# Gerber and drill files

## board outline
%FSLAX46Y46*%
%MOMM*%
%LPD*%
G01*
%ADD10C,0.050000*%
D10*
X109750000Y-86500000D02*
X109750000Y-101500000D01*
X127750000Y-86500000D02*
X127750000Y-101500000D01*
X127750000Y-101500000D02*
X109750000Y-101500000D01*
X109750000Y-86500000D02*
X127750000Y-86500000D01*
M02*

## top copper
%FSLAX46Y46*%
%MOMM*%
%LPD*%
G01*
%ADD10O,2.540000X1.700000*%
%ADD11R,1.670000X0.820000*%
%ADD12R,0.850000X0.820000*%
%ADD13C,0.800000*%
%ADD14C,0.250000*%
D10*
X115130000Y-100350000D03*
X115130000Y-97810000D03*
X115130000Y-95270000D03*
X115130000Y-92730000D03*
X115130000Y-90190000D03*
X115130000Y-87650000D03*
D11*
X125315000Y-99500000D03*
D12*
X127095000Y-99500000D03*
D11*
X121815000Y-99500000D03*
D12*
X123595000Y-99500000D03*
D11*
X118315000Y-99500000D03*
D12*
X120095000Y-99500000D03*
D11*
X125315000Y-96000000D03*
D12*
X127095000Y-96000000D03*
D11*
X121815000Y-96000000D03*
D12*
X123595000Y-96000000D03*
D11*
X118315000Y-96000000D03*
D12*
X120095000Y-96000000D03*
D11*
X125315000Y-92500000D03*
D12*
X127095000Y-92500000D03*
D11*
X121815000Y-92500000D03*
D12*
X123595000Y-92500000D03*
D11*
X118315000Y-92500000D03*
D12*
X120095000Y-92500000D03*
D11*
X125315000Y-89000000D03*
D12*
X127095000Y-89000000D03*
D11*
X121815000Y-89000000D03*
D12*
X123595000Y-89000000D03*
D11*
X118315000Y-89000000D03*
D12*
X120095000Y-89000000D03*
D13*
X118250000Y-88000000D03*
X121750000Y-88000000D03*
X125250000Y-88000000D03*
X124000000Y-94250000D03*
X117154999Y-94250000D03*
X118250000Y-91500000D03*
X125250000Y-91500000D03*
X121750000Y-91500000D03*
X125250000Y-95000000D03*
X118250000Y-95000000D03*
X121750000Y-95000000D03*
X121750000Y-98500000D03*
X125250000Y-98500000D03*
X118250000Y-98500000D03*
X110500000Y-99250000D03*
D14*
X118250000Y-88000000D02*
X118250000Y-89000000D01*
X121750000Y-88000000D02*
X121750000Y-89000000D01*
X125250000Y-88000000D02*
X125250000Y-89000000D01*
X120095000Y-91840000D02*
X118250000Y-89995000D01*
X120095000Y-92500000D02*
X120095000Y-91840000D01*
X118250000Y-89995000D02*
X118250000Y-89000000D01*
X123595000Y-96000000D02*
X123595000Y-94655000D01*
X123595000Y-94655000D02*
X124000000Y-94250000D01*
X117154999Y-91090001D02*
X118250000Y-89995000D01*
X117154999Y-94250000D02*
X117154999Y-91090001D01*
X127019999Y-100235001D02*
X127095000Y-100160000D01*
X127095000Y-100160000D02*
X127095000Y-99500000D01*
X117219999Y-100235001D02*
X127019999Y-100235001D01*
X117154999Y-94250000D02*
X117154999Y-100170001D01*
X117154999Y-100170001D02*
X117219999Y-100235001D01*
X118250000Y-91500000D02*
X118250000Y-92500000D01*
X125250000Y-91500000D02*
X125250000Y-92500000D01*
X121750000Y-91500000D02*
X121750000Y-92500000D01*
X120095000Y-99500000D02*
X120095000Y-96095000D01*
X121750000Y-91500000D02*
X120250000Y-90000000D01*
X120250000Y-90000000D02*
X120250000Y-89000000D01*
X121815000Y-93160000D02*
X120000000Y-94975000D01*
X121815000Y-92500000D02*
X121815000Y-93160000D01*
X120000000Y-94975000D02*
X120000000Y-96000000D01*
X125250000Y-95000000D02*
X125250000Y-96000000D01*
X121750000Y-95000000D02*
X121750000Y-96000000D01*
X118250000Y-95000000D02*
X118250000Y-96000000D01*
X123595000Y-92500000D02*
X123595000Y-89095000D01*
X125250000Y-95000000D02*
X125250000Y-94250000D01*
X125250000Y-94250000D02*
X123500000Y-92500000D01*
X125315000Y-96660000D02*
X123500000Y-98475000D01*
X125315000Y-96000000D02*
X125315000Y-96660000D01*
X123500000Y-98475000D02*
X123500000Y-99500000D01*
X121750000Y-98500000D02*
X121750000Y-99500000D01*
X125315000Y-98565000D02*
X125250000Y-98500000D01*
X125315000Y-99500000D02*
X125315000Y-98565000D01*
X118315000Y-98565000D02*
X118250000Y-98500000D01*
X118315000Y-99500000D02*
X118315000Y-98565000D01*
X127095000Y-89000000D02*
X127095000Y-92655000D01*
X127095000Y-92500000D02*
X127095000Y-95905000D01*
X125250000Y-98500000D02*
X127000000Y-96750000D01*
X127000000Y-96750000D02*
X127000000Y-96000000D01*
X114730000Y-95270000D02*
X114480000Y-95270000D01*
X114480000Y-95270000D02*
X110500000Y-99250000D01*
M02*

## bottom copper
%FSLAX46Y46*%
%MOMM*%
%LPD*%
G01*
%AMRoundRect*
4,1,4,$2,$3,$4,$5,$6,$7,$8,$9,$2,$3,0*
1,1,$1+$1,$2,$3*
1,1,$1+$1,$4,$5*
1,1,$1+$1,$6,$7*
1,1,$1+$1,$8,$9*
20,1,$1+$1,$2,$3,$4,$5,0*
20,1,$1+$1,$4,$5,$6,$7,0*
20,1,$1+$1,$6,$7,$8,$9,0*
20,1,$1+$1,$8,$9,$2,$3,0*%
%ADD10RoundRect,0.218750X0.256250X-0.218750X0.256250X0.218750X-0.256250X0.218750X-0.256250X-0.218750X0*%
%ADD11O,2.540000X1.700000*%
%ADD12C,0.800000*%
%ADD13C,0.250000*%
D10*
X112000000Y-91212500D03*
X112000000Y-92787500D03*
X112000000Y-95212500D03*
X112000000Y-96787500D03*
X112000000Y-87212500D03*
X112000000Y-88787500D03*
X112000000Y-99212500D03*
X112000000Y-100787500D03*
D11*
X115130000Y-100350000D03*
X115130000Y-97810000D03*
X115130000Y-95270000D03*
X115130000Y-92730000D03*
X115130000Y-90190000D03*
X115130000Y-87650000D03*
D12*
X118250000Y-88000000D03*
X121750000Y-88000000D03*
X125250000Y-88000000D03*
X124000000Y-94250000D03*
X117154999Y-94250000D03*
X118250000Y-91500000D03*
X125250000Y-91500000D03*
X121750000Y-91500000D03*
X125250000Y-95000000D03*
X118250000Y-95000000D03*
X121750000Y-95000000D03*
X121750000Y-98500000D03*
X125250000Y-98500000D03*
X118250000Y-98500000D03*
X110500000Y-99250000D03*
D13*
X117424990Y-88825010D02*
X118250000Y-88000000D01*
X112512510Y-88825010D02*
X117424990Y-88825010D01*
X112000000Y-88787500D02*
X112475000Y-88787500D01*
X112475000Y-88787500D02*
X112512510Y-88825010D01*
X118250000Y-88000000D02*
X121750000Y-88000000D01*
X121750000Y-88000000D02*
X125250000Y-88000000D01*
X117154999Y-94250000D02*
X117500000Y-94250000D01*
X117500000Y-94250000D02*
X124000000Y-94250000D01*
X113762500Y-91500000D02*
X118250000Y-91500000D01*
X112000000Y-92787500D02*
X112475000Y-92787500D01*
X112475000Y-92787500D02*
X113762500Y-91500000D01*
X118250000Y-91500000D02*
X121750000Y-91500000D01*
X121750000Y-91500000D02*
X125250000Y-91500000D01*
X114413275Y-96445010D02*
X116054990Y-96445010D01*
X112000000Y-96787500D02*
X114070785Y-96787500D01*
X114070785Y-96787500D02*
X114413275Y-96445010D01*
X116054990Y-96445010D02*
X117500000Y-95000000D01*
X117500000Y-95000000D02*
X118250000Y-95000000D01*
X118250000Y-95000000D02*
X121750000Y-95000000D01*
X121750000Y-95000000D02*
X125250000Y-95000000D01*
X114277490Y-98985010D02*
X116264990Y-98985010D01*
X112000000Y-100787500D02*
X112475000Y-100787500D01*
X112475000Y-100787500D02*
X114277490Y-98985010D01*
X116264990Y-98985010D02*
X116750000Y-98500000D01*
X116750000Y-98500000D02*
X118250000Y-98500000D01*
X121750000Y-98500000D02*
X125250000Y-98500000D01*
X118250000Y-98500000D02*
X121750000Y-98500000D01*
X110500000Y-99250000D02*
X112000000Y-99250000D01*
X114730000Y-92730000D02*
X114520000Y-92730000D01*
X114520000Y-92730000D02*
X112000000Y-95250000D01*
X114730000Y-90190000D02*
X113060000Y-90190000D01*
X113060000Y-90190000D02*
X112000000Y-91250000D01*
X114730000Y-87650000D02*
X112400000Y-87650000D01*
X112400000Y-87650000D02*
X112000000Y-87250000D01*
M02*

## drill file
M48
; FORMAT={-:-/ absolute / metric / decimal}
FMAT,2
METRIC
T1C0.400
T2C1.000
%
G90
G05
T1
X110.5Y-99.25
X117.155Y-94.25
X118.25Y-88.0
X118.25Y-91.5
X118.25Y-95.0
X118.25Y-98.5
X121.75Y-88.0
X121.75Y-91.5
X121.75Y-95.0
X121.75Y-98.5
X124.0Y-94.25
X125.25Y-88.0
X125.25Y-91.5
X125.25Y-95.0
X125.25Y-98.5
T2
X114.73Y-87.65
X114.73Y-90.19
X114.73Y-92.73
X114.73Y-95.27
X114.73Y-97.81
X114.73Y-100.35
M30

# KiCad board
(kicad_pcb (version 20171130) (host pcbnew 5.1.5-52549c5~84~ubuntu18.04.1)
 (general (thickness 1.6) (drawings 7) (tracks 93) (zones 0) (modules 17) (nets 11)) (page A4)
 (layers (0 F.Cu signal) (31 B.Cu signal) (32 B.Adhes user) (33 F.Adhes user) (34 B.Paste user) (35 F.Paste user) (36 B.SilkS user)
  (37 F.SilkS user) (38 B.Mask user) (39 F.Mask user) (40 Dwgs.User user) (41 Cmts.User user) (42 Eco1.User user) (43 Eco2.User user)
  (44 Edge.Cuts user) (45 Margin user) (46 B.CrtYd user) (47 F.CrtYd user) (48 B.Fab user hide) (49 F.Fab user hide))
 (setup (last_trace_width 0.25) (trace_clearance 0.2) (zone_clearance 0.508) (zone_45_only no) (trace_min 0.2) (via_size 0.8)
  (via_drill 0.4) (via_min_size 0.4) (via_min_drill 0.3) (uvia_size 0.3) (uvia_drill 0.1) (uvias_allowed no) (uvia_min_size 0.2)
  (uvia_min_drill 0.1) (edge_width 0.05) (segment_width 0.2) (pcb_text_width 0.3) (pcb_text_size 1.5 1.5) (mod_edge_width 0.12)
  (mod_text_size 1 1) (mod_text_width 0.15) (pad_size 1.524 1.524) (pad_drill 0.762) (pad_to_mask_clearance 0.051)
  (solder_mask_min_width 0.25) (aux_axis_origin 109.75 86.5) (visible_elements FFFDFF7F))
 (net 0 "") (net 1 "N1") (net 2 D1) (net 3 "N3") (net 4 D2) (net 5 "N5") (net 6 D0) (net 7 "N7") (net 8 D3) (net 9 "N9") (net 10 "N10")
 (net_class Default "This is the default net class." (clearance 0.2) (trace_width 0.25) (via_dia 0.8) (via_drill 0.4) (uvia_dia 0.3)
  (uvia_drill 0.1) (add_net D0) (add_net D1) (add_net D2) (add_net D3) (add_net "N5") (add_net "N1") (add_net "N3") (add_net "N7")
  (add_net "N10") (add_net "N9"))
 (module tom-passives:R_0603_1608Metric (layer B.Cu) (at 112 92 90)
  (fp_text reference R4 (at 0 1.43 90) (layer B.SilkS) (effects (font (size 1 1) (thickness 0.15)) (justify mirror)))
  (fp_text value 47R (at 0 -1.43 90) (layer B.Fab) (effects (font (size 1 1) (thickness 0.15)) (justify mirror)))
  (pad 2 smd roundrect (at 0.7875 0 90) (size 0.875 0.95) (layers B.Cu B.Paste B.Mask) (roundrect_rratio 0.25) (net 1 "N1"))
  (pad 1 smd roundrect (at -0.7875 0 90) (size 0.875 0.95) (layers B.Cu B.Paste B.Mask) (roundrect_rratio 0.25) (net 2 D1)))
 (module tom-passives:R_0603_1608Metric (layer B.Cu) (at 112 96 90)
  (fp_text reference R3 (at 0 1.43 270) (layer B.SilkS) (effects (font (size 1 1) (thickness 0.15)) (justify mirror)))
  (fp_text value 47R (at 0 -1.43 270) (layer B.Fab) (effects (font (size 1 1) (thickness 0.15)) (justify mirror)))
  (pad 2 smd roundrect (at 0.7875 0 90) (size 0.875 0.95) (layers B.Cu B.Paste B.Mask) (roundrect_rratio 0.25) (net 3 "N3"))
  (pad 1 smd roundrect (at -0.7875 0 90) (size 0.875 0.95) (layers B.Cu B.Paste B.Mask) (roundrect_rratio 0.25) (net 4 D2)))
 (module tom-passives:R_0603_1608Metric (layer B.Cu) (at 112 88 90)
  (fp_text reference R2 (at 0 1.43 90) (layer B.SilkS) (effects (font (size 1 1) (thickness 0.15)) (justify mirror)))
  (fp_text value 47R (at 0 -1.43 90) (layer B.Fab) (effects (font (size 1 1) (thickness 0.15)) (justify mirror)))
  (pad 2 smd roundrect (at 0.7875 0 90) (size 0.875 0.95) (layers B.Cu B.Paste B.Mask) (roundrect_rratio 0.25) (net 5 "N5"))
  (pad 1 smd roundrect (at -0.7875 0 90) (size 0.875 0.95) (layers B.Cu B.Paste B.Mask) (roundrect_rratio 0.25) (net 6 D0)))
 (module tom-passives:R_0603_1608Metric (layer B.Cu) (at 112 100 90)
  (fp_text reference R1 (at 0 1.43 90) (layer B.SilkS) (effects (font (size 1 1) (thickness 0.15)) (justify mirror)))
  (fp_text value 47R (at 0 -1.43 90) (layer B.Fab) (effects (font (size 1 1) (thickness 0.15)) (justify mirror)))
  (pad 2 smd roundrect (at 0.7875 0 90) (size 0.875 0.95) (layers B.Cu B.Paste B.Mask) (roundrect_rratio 0.25) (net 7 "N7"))
  (pad 1 smd roundrect (at -0.7875 0 90) (size 0.875 0.95) (layers B.Cu B.Paste B.Mask) (roundrect_rratio 0.25) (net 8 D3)))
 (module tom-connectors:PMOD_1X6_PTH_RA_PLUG (layer F.Cu) (at 116 94 270)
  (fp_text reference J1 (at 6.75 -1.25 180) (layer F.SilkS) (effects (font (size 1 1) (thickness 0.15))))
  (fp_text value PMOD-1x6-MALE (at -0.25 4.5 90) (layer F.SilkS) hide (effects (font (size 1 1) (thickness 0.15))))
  (pad 6 thru_hole oval (at 6.35 1.27 180) (size 2.54 1.7) (drill 1 (offset -0.4 0)) (layers *.Cu *.Mask) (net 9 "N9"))
  (pad 5 thru_hole oval (at 3.81 1.27 180) (size 2.54 1.7) (drill 1 (offset -0.4 0)) (layers *.Cu *.Mask) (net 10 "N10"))
  (pad 4 thru_hole oval (at 1.27 1.27 180) (size 2.54 1.7) (drill 1 (offset -0.4 0)) (layers *.Cu *.Mask) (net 7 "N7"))
  (pad 3 thru_hole oval (at -1.27 1.27 180) (size 2.54 1.7) (drill 1 (offset -0.4 0)) (layers *.Cu *.Mask) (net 3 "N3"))
  (pad 2 thru_hole oval (at -3.81 1.27 180) (size 2.54 1.7) (drill 1 (offset -0.4 0)) (layers *.Cu *.Mask) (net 1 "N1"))
  (pad 1 thru_hole oval (at -6.35 1.27 180) (size 2.54 1.7) (drill 1 (offset -0.4 0)) (layers *.Cu *.Mask) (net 5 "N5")))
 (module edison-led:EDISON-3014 (layer F.Cu) (at 126 99.5)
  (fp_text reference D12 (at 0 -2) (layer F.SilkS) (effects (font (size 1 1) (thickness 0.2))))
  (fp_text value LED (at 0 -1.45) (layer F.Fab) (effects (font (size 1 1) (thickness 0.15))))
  (pad 2 smd rect (at -0.685 0) (size 1.67 0.82) (layers F.Cu F.Paste F.Mask) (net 8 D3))
  (pad 1 smd rect (at 1.095 0) (size 0.85 0.82) (layers F.Cu F.Paste F.Mask) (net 6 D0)))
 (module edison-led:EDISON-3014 (layer F.Cu) (at 122.5 99.5)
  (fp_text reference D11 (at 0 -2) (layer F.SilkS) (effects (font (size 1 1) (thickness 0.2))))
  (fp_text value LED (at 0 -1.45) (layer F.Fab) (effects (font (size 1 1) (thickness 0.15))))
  (pad 2 smd rect (at -0.685 0) (size 1.67 0.82) (layers F.Cu F.Paste F.Mask) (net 8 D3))
  (pad 1 smd rect (at 1.095 0) (size 0.85 0.82) (layers F.Cu F.Paste F.Mask) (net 4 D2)))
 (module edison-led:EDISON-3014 (layer F.Cu) (at 119 99.5)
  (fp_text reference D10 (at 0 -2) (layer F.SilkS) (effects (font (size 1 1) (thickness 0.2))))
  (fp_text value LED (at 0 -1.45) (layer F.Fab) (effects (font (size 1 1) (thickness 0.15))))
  (pad 2 smd rect (at -0.685 0) (size 1.67 0.82) (layers F.Cu F.Paste F.Mask) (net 8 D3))
  (pad 1 smd rect (at 1.095 0) (size 0.85 0.82) (layers F.Cu F.Paste F.Mask) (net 2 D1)))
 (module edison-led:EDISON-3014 (layer F.Cu) (at 126 96)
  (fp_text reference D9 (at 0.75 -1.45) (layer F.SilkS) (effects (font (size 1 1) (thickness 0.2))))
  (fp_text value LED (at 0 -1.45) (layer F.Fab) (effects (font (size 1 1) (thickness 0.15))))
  (pad 2 smd rect (at -0.685 0) (size 1.67 0.82) (layers F.Cu F.Paste F.Mask) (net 4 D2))
  (pad 1 smd rect (at 1.095 0) (size 0.85 0.82) (layers F.Cu F.Paste F.Mask) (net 8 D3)))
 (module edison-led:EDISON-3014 (layer F.Cu) (at 122.5 96)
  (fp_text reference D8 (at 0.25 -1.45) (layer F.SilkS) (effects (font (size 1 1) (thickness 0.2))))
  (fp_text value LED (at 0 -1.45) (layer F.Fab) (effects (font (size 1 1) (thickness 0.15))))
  (pad 2 smd rect (at -0.685 0) (size 1.67 0.82) (layers F.Cu F.Paste F.Mask) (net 4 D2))
  (pad 1 smd rect (at 1.095 0) (size 0.85 0.82) (layers F.Cu F.Paste F.Mask) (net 6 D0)))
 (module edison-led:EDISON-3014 (layer F.Cu) (at 119 96)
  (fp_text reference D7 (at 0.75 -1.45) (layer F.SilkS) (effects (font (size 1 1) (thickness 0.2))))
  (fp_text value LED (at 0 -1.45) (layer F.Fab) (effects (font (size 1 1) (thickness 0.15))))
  (pad 2 smd rect (at -0.685 0) (size 1.67 0.82) (layers F.Cu F.Paste F.Mask) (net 4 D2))
  (pad 1 smd rect (at 1.095 0) (size 0.85 0.82) (layers F.Cu F.Paste F.Mask) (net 2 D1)))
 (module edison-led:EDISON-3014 (layer F.Cu) (at 126 92.5)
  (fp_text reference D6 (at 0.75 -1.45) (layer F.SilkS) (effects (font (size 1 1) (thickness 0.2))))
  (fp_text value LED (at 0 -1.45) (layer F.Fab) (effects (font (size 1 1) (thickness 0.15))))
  (pad 2 smd rect (at -0.685 0) (size 1.67 0.82) (layers F.Cu F.Paste F.Mask) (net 2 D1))
  (pad 1 smd rect (at 1.095 0) (size 0.85 0.82) (layers F.Cu F.Paste F.Mask) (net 8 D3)))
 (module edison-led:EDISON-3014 (layer F.Cu) (at 122.5 92.5)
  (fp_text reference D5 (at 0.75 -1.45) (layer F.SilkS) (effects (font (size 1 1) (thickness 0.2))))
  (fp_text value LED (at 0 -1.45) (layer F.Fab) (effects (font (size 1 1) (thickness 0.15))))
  (pad 2 smd rect (at -0.685 0) (size 1.67 0.82) (layers F.Cu F.Paste F.Mask) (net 2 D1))
  (pad 1 smd rect (at 1.095 0) (size 0.85 0.82) (layers F.Cu F.Paste F.Mask) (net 4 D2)))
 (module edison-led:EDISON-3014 (layer F.Cu) (at 119 92.5)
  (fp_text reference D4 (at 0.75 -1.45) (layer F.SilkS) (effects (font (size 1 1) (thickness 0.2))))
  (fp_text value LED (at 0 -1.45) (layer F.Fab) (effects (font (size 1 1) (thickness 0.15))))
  (pad 2 smd rect (at -0.685 0) (size 1.67 0.82) (layers F.Cu F.Paste F.Mask) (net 2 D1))
  (pad 1 smd rect (at 1.095 0) (size 0.85 0.82) (layers F.Cu F.Paste F.Mask) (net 6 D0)))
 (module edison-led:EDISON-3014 (layer F.Cu) (at 126 89)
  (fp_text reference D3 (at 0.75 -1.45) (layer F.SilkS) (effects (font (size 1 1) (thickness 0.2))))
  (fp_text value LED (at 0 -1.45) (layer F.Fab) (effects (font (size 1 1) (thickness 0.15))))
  (pad 2 smd rect (at -0.685 0) (size 1.67 0.82) (layers F.Cu F.Paste F.Mask) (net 6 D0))
  (pad 1 smd rect (at 1.095 0) (size 0.85 0.82) (layers F.Cu F.Paste F.Mask) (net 8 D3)))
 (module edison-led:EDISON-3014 (layer F.Cu) (at 122.5 89)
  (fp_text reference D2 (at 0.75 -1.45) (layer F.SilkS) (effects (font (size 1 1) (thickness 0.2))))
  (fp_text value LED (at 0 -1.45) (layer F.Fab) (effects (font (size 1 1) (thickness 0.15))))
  (pad 2 smd rect (at -0.685 0) (size 1.67 0.82) (layers F.Cu F.Paste F.Mask) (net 6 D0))
  (pad 1 smd rect (at 1.095 0) (size 0.85 0.82) (layers F.Cu F.Paste F.Mask) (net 4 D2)))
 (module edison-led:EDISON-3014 (layer F.Cu) (at 119 89)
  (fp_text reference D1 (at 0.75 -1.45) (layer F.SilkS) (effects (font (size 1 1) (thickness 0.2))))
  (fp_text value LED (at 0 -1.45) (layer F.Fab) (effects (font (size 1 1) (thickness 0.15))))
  (pad 2 smd rect (at -0.685 0) (size 1.67 0.82) (layers F.Cu F.Paste F.Mask) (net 6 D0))
  (pad 1 smd rect (at 1.095 0) (size 0.85 0.82) (layers F.Cu F.Paste F.Mask) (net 2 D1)))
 (gr_line (start 109.75 86.5) (end 109.75 101.5) (layer Edge.Cuts) (width 0.05))
 (gr_line (start 127.75 86.5) (end 127.75 101.5) (layer Edge.Cuts) (width 0.05))
 (gr_line (start 127.75 101.5) (end 109.75 101.5) (layer Edge.Cuts) (width 0.05))
 (gr_line (start 109.75 86.5) (end 127.75 86.5) (layer Edge.Cuts) (width 0.05))
 (segment (start 117.42499 88.82501) (end 118.25 88) (width 0.25) (layer B.Cu) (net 6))
 (segment (start 112.51251 88.82501) (end 117.42499 88.82501) (width 0.25) (layer B.Cu) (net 6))
 (via (at 118.25 88) (size 0.8) (drill 0.4) (layers F.Cu B.Cu) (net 6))
 (segment (start 112 88.7875) (end 112.475 88.7875) (width 0.25) (layer B.Cu) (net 6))
 (segment (start 112.475 88.7875) (end 112.51251 88.82501) (width 0.25) (layer B.Cu) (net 6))
 (segment (start 118.25 88) (end 118.25 89) (width 0.25) (layer F.Cu) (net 6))
 (via (at 121.75 88) (size 0.8) (drill 0.4) (layers F.Cu B.Cu) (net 6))
 (segment (start 118.25 88) (end 121.75 88) (width 0.25) (layer B.Cu) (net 6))
 (segment (start 121.75 88) (end 121.75 89) (width 0.25) (layer F.Cu) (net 6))
 (via (at 125.25 88) (size 0.8) (drill 0.4) (layers F.Cu B.Cu) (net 6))
 (segment (start 121.75 88) (end 125.25 88) (width 0.25) (layer B.Cu) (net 6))
 (segment (start 125.25 88) (end 125.25 89) (width 0.25) (layer F.Cu) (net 6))
 (segment (start 120.095 91.84) (end 118.25 89.995) (width 0.25) (layer F.Cu) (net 6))
 (segment (start 120.095 92.5) (end 120.095 91.84) (width 0.25) (layer F.Cu) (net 6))
 (segment (start 118.25 89.995) (end 118.25 89) (width 0.25) (layer F.Cu) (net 6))
 (via (at 124 94.25) (size 0.8) (drill 0.4) (layers F.Cu B.Cu) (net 6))
 (segment (start 123.595 96) (end 123.595 94.655) (width 0.25) (layer F.Cu) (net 6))
 (segment (start 123.595 94.655) (end 124 94.25) (width 0.25) (layer F.Cu) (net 6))
 (segment (start 117.154999 91.090001) (end 118.25 89.995) (width 0.25) (layer F.Cu) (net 6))
 (segment (start 117.154999 94.25) (end 117.154999 91.090001) (width 0.25) (layer F.Cu) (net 6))
 (segment (start 127.019999 100.235001) (end 127.095 100.16) (width 0.25) (layer F.Cu) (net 6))
 (segment (start 117.154999 94.25) (end 117.5 94.25) (width 0.25) (layer B.Cu) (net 6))
 (via (at 117.154999 94.25) (size 0.8) (drill 0.4) (layers F.Cu B.Cu) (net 6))
 (segment (start 127.095 100.16) (end 127.095 99.5) (width 0.25) (layer F.Cu) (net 6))
 (segment (start 117.219999 100.235001) (end 127.019999 100.235001) (width 0.25) (layer F.Cu) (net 6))
 (segment (start 117.5 94.25) (end 124 94.25) (width 0.25) (layer B.Cu) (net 6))
 (segment (start 117.154999 94.25) (end 117.154999 100.170001) (width 0.25) (layer F.Cu) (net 6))
 (segment (start 117.154999 100.170001) (end 117.219999 100.235001) (width 0.25) (layer F.Cu) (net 6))
 (segment (start 113.7625 91.5) (end 118.25 91.5) (width 0.25) (layer B.Cu) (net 2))
 (segment (start 112 92.7875) (end 112.475 92.7875) (width 0.25) (layer B.Cu) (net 2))
 (via (at 118.25 91.5) (size 0.8) (drill 0.4) (layers F.Cu B.Cu) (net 2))
 (segment (start 112.475 92.7875) (end 113.7625 91.5) (width 0.25) (layer B.Cu) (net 2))
 (segment (start 118.25 91.5) (end 118.25 92.5) (width 0.25) (layer F.Cu) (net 2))
 (segment (start 118.25 91.5) (end 121.75 91.5) (width 0.25) (layer B.Cu) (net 2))
 (via (at 125.25 91.5) (size 0.8) (drill 0.4) (layers F.Cu B.Cu) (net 2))
 (segment (start 125.25 91.5) (end 125.25 92.5) (width 0.25) (layer F.Cu) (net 2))
 (segment (start 121.75 91.5) (end 125.25 91.5) (width 0.25) (layer B.Cu) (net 2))
 (via (at 121.75 91.5) (size 0.8) (drill 0.4) (layers F.Cu B.Cu) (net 2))
 (segment (start 121.75 91.5) (end 121.75 92.5) (width 0.25) (layer F.Cu) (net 2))
 (segment (start 120.095 99.5) (end 120.095 96.095) (width 0.25) (layer F.Cu) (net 2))
 (segment (start 121.75 91.5) (end 120.25 90) (width 0.25) (layer F.Cu) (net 2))
 (segment (start 120.25 90) (end 120.25 89) (width 0.25) (layer F.Cu) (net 2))
 (segment (start 121.815 93.16) (end 120 94.975) (width 0.25) (layer F.Cu) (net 2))
 (segment (start 121.815 92.5) (end 121.815 93.16) (width 0.25) (layer F.Cu) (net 2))
 (segment (start 120 94.975) (end 120 96) (width 0.25) (layer F.Cu) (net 2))
 (segment (start 114.413275 96.44501) (end 116.05499 96.44501) (width 0.25) (layer B.Cu) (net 4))
 (segment (start 112 96.7875) (end 114.070785 96.7875) (width 0.25) (layer B.Cu) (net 4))
 (segment (start 114.070785 96.7875) (end 114.413275 96.44501) (width 0.25) (layer B.Cu) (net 4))
 (segment (start 116.05499 96.44501) (end 117.5 95) (width 0.25) (layer B.Cu) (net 4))
 (via (at 125.25 95) (size 0.8) (drill 0.4) (layers F.Cu B.Cu) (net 4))
 (segment (start 117.5 95) (end 118.25 95) (width 0.25) (layer B.Cu) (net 4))
 (segment (start 125.25 95) (end 125.25 96) (width 0.25) (layer F.Cu) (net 4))
 (segment (start 118.25 95) (end 121.75 95) (width 0.25) (layer B.Cu) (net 4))
 (via (at 118.25 95) (size 0.8) (drill 0.4) (layers F.Cu B.Cu) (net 4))
 (segment (start 121.75 95) (end 125.25 95) (width 0.25) (layer B.Cu) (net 4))
 (via (at 121.75 95) (size 0.8) (drill 0.4) (layers F.Cu B.Cu) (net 4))
 (segment (start 121.75 95) (end 121.75 96) (width 0.25) (layer F.Cu) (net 4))
 (segment (start 118.25 95) (end 118.25 96) (width 0.25) (layer F.Cu) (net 4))
 (segment (start 123.595 92.5) (end 123.595 89.095) (width 0.25) (layer F.Cu) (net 4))
 (segment (start 125.25 95) (end 125.25 94.25) (width 0.25) (layer F.Cu) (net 4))
 (segment (start 125.25 94.25) (end 123.5 92.5) (width 0.25) (layer F.Cu) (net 4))
 (segment (start 125.315 96.66) (end 123.5 98.475) (width 0.25) (layer F.Cu) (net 4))
 (segment (start 125.315 96) (end 125.315 96.66) (width 0.25) (layer F.Cu) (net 4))
 (segment (start 123.5 98.475) (end 123.5 99.5) (width 0.25) (layer F.Cu) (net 4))
 (segment (start 114.27749 98.98501) (end 116.26499 98.98501) (width 0.25) (layer B.Cu) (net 8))
 (segment (start 112 100.7875) (end 112.475 100.7875) (width 0.25) (layer B.Cu) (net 8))
 (segment (start 112.475 100.7875) (end 114.27749 98.98501) (width 0.25) (layer B.Cu) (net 8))
 (via (at 121.75 98.5) (size 0.8) (drill 0.4) (layers F.Cu B.Cu) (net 8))
 (segment (start 116.26499 98.98501) (end 116.75 98.5) (width 0.25) (layer B.Cu) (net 8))
 (segment (start 116.75 98.5) (end 118.25 98.5) (width 0.25) (layer B.Cu) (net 8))
 (segment (start 121.75 98.5) (end 121.75 99.5) (width 0.25) (layer F.Cu) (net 8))
 (segment (start 121.75 98.5) (end 125.25 98.5) (width 0.25) (layer B.Cu) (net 8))
 (via (at 125.25 98.5) (size 0.8) (drill 0.4) (layers F.Cu B.Cu) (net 8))
 (segment (start 125.315 98.565) (end 125.25 98.5) (width 0.25) (layer F.Cu) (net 8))
 (segment (start 125.315 99.5) (end 125.315 98.565) (width 0.25) (layer F.Cu) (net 8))
 (segment (start 118.25 98.5) (end 121.75 98.5) (width 0.25) (layer B.Cu) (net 8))
 (via (at 118.25 98.5) (size 0.8) (drill 0.4) (layers F.Cu B.Cu) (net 8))
 (segment (start 118.315 98.565) (end 118.25 98.5) (width 0.25) (layer F.Cu) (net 8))
 (segment (start 118.315 99.5) (end 118.315 98.565) (width 0.25) (layer F.Cu) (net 8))
 (segment (start 127.095 89) (end 127.095 92.655) (width 0.25) (layer F.Cu) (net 8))
 (segment (start 127.095 92.5) (end 127.095 95.905) (width 0.25) (layer F.Cu) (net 8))
 (segment (start 125.25 98.5) (end 127 96.75) (width 0.25) (layer F.Cu) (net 8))
 (segment (start 127 96.75) (end 127 96) (width 0.25) (layer F.Cu) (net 8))
 (via (at 110.5 99.25) (size 0.8) (drill 0.4) (layers F.Cu B.Cu) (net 7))
 (segment (start 114.73 95.27) (end 114.48 95.27) (width 0.25) (layer F.Cu) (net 7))
 (segment (start 114.48 95.27) (end 110.5 99.25) (width 0.25) (layer F.Cu) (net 7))
 (segment (start 110.5 99.25) (end 112 99.25) (width 0.25) (layer B.Cu) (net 7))
 (segment (start 114.73 92.73) (end 114.52 92.73) (width 0.25) (layer B.Cu) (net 3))
 (segment (start 114.52 92.73) (end 112 95.25) (width 0.25) (layer B.Cu) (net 3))
 (segment (start 114.73 90.19) (end 113.06 90.19) (width 0.25) (layer B.Cu) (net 1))
 (segment (start 113.06 90.19) (end 112 91.25) (width 0.25) (layer B.Cu) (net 1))
 (segment (start 114.73 87.65) (end 112.4 87.65) (width 0.25) (layer B.Cu) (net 5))
 (segment (start 112.4 87.65) (end 112 87.25) (width 0.25) (layer B.Cu) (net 5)))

